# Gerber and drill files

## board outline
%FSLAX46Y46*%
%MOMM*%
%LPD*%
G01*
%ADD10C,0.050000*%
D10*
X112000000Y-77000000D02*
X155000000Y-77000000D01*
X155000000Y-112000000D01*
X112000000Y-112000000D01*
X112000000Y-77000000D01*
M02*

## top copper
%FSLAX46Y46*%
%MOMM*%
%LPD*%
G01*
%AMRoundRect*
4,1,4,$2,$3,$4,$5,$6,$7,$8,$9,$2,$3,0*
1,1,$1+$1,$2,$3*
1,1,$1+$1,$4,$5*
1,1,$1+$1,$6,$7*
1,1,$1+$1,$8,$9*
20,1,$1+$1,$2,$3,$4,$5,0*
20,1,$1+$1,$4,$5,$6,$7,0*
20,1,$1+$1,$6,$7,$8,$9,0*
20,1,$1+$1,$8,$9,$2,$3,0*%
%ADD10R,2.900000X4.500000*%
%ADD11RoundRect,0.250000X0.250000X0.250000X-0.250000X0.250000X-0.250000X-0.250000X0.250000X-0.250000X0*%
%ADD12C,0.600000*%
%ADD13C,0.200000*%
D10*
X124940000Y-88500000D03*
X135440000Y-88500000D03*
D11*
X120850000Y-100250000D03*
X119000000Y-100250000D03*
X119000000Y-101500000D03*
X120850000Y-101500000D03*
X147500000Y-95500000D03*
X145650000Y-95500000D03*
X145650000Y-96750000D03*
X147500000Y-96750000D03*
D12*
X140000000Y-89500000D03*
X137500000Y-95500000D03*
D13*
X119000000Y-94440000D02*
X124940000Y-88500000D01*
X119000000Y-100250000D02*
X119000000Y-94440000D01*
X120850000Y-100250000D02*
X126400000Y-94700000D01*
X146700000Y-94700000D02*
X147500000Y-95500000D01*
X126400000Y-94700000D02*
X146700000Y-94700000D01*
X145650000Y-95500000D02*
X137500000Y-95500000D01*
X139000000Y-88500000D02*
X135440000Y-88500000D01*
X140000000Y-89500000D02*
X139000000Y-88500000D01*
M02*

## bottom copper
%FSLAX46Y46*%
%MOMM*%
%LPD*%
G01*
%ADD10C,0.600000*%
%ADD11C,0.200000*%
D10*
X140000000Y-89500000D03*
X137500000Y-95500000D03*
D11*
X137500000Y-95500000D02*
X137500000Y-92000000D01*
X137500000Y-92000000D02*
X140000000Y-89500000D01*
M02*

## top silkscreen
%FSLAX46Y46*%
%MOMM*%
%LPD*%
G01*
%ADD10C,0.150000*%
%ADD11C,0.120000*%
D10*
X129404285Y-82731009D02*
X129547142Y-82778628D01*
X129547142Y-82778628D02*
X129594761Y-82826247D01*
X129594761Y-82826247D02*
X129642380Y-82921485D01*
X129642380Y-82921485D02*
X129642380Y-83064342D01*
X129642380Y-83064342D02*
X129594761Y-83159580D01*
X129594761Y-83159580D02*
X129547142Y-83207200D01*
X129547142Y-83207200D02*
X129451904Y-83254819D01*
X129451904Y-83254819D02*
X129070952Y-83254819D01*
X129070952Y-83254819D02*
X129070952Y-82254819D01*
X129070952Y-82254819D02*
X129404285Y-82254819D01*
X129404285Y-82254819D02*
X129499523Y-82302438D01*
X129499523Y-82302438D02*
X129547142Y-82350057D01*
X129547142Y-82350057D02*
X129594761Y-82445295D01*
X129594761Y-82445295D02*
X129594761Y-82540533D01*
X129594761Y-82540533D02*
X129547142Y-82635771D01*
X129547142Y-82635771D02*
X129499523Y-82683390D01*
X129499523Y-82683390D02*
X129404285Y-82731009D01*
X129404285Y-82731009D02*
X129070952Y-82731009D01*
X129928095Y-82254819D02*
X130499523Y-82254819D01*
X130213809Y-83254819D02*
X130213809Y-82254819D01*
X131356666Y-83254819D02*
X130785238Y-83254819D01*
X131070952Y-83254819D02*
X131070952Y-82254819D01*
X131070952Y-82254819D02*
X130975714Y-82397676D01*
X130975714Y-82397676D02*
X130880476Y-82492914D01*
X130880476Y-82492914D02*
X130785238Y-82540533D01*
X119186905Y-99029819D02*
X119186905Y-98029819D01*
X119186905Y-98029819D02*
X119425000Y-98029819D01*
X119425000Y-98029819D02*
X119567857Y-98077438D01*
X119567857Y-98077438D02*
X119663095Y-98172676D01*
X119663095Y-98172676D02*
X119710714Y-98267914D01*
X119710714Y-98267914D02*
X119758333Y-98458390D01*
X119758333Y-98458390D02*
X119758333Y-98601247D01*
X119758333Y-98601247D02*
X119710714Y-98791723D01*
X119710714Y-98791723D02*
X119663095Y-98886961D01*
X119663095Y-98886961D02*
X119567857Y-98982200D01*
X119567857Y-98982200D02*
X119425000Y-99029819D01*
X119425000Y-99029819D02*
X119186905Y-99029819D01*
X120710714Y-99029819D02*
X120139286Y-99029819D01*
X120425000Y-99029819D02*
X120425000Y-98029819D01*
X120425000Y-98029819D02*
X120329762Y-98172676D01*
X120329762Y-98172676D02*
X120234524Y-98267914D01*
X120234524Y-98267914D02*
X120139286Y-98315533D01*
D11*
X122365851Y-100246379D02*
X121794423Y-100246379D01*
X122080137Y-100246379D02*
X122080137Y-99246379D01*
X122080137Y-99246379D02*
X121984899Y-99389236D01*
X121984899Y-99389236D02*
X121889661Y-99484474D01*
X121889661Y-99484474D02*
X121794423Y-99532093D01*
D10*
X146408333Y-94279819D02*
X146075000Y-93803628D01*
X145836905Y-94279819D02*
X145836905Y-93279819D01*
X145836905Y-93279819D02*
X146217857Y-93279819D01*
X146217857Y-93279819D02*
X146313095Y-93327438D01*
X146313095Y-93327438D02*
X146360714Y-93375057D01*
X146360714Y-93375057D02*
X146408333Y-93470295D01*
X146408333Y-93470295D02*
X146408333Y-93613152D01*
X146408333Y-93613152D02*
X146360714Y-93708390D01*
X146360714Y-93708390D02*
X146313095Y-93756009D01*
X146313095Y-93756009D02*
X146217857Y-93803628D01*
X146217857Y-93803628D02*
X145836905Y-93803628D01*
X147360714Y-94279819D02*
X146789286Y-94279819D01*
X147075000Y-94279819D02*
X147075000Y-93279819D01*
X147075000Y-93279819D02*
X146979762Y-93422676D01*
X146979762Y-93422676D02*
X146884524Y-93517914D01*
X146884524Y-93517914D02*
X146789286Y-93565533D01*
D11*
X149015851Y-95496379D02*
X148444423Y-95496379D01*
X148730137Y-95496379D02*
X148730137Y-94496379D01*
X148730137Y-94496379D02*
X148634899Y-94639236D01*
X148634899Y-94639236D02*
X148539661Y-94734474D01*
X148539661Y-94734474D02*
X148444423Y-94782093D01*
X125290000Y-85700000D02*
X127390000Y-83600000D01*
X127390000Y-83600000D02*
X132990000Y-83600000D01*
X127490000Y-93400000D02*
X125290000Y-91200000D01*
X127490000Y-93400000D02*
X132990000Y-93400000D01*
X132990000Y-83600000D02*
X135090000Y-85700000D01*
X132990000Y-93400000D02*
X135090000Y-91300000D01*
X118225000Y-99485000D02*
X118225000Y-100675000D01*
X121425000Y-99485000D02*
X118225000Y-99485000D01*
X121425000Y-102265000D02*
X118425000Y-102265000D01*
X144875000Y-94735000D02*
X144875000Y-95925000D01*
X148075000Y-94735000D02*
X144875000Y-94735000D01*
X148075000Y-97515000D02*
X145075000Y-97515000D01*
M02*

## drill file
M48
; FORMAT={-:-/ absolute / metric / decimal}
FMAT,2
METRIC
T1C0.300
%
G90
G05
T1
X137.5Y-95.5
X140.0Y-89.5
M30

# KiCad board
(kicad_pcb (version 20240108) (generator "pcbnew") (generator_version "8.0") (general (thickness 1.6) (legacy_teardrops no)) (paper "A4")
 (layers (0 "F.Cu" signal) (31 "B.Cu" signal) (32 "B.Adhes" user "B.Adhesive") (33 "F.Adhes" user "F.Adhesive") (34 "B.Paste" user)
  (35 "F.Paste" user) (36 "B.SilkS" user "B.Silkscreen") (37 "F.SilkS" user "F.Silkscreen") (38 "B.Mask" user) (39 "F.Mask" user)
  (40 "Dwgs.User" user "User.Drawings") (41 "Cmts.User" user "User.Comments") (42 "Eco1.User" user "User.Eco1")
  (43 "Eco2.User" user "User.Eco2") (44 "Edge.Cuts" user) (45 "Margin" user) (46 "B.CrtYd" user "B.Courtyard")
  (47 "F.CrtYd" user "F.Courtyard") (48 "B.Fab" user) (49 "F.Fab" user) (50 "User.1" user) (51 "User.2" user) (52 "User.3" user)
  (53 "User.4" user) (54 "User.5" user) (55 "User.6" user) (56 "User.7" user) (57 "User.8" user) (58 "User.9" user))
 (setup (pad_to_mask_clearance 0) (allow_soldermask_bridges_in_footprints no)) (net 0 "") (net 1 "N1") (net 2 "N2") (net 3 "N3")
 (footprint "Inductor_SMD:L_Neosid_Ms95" (layer "F.Cu") (at 130.19 88.5)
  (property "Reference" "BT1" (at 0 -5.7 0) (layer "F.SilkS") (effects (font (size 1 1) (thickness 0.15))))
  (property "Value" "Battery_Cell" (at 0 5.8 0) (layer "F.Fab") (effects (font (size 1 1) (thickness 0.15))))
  (fp_line (start -4.9 -2.8) (end -2.8 -4.9) (stroke (width 0.12) (type solid)) (layer "F.SilkS"))
  (fp_line (start -2.8 -4.9) (end 2.8 -4.9) (stroke (width 0.12) (type solid)) (layer "F.SilkS"))
  (fp_line (start -2.7 4.9) (end -4.9 2.7) (stroke (width 0.12) (type solid)) (layer "F.SilkS"))
  (fp_line (start -2.7 4.9) (end 2.8 4.9) (stroke (width 0.12) (type solid)) (layer "F.SilkS"))
  (fp_line (start 2.8 -4.9) (end 4.9 -2.8) (stroke (width 0.12) (type solid)) (layer "F.SilkS"))
  (fp_line (start 2.8 4.9) (end 4.9 2.8) (stroke (width 0.12) (type solid)) (layer "F.SilkS"))
  (pad "1" smd rect (at -5.25 0) (size 2.9 4.5) (layers "F.Cu" "F.Paste" "F.Mask") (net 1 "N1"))
  (pad "2" smd rect (at 5.25 0) (size 2.9 4.5) (layers "F.Cu" "F.Paste" "F.Mask") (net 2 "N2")))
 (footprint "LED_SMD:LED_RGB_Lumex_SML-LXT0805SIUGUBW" (layer "F.Cu") (at 119.925 100.875)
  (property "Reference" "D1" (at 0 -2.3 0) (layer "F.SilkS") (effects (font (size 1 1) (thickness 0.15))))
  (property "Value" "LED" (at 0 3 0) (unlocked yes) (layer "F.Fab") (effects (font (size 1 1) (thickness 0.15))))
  (fp_line (start -1.7 -1.39) (end -1.7 -0.2) (stroke (width 0.12) (type default)) (layer "F.SilkS"))
  (fp_line (start 1.5 -1.39) (end -1.7 -1.39) (stroke (width 0.12) (type solid)) (layer "F.SilkS"))
  (fp_line (start 1.5 1.39) (end -1.5 1.39) (stroke (width 0.12) (type solid)) (layer "F.SilkS"))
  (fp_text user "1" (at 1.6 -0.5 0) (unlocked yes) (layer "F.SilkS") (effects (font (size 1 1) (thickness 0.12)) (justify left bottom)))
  (pad "1" smd roundrect (at 0.925 -0.625 180) (size 1 1) (layers "F.Cu" "F.Paste" "F.Mask") (roundrect_rratio 0.25) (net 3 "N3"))
  (pad "2" smd roundrect (at -0.925 -0.625 180) (size 1 1) (layers "F.Cu" "F.Paste" "F.Mask") (roundrect_rratio 0.25) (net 1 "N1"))
  (pad "3" smd roundrect (at -0.925 0.625 180) (size 1 1) (layers "F.Cu" "F.Paste" "F.Mask") (roundrect_rratio 0.25))
  (pad "4" smd roundrect (at 0.925 0.625 180) (size 1 1) (layers "F.Cu" "F.Paste" "F.Mask") (roundrect_rratio 0.25)))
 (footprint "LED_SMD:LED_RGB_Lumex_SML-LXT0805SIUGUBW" (layer "F.Cu") (at 146.575 96.125)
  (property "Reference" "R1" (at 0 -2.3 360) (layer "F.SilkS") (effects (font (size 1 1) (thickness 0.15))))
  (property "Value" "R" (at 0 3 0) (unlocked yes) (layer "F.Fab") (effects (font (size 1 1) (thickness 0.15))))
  (fp_line (start -1.7 -1.39) (end -1.7 -0.2) (stroke (width 0.12) (type default)) (layer "F.SilkS"))
  (fp_line (start 1.5 -1.39) (end -1.7 -1.39) (stroke (width 0.12) (type solid)) (layer "F.SilkS"))
  (fp_line (start 1.5 1.39) (end -1.5 1.39) (stroke (width 0.12) (type solid)) (layer "F.SilkS"))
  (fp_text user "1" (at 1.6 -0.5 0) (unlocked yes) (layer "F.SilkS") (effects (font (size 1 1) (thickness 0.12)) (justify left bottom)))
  (pad "1" smd roundrect (at 0.925 -0.625 180) (size 1 1) (layers "F.Cu" "F.Paste" "F.Mask") (roundrect_rratio 0.25) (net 3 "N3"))
  (pad "2" smd roundrect (at -0.925 -0.625 180) (size 1 1) (layers "F.Cu" "F.Paste" "F.Mask") (roundrect_rratio 0.25) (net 2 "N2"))
  (pad "3" smd roundrect (at -0.925 0.625 180) (size 1 1) (layers "F.Cu" "F.Paste" "F.Mask") (roundrect_rratio 0.25))
  (pad "4" smd roundrect (at 0.925 0.625 180) (size 1 1) (layers "F.Cu" "F.Paste" "F.Mask") (roundrect_rratio 0.25)))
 (gr_rect (start 112 77) (end 155 112) (stroke (width 0.05) (type default)) (fill none) (layer "Edge.Cuts"))
 (segment (start 119 94.44) (end 124.94 88.5) (width 0.2) (layer "F.Cu") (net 1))
 (segment (start 119 100.25) (end 119 94.44) (width 0.2) (layer "F.Cu") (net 1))
 (segment (start 120.85 100.25) (end 126.4 94.7) (width 0.2) (layer "F.Cu") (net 3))
 (segment (start 146.7 94.7) (end 147.5 95.5) (width 0.2) (layer "F.Cu") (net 3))
 (segment (start 126.4 94.7) (end 146.7 94.7) (width 0.2) (layer "F.Cu") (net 3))
 (segment (start 145.65 95.5) (end 137.5 95.5) (width 0.2) (layer "F.Cu") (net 2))
 (segment (start 139 88.5) (end 135.44 88.5) (width 0.2) (layer "F.Cu") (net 2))
 (segment (start 140 89.5) (end 139 88.5) (width 0.2) (layer "F.Cu") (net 2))
 (via (at 140 89.5) (size 0.6) (drill 0.3) (layers "F.Cu" "B.Cu") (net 2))
 (via (at 137.5 95.5) (size 0.6) (drill 0.3) (layers "F.Cu" "B.Cu") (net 2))
 (segment (start 137.5 95.5) (end 137.5 92) (width 0.2) (layer "B.Cu") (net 2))
 (segment (start 137.5 92) (end 140 89.5) (width 0.2) (layer "B.Cu") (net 2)))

